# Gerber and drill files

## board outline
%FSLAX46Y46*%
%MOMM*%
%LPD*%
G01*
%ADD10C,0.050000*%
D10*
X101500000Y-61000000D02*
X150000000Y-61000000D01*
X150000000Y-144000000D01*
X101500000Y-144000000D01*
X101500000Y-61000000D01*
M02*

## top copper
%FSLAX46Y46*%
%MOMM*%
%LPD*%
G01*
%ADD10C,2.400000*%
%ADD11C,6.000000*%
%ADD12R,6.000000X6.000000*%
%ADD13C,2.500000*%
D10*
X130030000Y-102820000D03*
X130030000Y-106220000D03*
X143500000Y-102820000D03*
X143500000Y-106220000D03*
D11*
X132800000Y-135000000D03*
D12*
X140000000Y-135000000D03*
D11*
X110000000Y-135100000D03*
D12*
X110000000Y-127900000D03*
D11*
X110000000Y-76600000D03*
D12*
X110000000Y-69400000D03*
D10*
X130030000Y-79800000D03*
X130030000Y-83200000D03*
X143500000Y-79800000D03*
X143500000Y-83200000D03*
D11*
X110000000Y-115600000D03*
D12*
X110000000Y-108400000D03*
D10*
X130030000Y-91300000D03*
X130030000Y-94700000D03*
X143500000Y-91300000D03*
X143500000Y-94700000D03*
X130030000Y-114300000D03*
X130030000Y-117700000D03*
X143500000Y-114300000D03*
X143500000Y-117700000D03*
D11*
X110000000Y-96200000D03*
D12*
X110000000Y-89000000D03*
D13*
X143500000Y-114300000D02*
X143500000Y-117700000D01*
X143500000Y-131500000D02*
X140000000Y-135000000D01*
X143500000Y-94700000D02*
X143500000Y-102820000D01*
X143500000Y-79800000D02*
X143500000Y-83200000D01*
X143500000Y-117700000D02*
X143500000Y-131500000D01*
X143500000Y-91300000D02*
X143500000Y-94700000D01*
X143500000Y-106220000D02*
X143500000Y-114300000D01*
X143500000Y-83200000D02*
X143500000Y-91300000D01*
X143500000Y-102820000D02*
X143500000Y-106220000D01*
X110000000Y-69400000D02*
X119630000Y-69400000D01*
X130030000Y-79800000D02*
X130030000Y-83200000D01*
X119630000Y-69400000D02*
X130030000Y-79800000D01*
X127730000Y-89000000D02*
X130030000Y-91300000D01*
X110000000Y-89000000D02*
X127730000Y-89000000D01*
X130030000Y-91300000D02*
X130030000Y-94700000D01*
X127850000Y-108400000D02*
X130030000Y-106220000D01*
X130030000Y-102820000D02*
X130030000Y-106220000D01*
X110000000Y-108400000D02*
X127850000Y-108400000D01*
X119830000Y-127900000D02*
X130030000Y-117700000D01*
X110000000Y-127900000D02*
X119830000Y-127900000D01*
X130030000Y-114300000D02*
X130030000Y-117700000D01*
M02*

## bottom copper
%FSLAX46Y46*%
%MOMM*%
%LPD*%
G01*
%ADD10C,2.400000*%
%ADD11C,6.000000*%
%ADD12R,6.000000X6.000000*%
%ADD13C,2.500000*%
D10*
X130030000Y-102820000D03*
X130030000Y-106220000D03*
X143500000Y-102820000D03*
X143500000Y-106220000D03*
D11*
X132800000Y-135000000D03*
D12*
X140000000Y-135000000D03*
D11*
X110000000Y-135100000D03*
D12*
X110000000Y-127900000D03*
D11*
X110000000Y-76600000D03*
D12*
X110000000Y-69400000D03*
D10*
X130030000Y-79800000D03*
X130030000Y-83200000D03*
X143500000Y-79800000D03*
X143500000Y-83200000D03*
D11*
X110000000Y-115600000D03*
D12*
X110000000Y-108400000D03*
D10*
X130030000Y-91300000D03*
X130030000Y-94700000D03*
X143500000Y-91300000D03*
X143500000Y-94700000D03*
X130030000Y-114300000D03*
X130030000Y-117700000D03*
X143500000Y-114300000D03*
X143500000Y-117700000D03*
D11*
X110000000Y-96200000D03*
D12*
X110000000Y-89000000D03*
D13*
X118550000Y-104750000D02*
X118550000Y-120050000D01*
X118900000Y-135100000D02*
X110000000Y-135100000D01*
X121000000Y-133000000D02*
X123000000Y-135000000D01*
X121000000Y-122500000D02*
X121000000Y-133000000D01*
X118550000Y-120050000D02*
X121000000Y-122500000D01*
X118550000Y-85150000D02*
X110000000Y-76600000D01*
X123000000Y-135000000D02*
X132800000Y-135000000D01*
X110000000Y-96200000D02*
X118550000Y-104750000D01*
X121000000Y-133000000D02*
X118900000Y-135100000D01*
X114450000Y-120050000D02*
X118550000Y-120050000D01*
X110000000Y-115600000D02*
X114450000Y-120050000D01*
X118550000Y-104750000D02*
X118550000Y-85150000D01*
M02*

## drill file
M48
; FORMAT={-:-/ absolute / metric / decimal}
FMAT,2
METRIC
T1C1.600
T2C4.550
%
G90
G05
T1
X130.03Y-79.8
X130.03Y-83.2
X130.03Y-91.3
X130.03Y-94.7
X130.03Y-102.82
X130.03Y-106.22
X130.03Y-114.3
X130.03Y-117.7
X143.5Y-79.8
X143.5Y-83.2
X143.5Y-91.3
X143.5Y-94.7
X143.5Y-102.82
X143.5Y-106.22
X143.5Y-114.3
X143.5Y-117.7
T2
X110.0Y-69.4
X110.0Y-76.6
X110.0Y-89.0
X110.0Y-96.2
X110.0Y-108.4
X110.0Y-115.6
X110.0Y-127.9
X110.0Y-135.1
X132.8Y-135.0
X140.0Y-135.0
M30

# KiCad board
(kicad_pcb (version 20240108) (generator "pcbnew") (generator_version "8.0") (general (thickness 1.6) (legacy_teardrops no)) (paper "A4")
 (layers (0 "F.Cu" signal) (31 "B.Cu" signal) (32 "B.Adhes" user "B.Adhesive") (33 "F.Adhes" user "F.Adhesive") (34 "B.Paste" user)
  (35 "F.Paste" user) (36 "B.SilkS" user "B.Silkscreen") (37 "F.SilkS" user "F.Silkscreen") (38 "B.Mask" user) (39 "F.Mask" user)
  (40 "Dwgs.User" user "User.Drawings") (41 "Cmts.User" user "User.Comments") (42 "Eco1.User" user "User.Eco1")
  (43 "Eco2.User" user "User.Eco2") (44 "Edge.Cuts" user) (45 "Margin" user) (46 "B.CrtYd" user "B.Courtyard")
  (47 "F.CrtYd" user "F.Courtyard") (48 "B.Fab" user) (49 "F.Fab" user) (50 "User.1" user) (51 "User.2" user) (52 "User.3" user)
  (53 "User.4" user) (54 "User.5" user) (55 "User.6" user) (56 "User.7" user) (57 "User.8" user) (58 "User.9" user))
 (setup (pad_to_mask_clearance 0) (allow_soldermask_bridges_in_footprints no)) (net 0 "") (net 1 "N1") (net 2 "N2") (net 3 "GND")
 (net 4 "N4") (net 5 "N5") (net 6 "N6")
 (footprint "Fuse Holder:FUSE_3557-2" (layer "F.Cu") (at 136.765 104.52)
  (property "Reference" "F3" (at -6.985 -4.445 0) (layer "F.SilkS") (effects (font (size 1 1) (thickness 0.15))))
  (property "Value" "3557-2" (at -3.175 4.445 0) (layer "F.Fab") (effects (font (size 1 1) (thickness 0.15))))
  (pad "1_1" thru_hole circle (at -6.735 -1.7) (size 2.4 2.4) (drill 1.6) (layers "*.Cu" "*.Mask") (remove_unused_layers no) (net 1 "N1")
   (solder_mask_margin 0.102))
  (pad "1_2" thru_hole circle (at -6.735 1.7) (size 2.4 2.4) (drill 1.6) (layers "*.Cu" "*.Mask") (remove_unused_layers no) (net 1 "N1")
   (solder_mask_margin 0.102))
  (pad "2_1" thru_hole circle (at 6.735 -1.7) (size 2.4 2.4) (drill 1.6) (layers "*.Cu" "*.Mask") (remove_unused_layers no) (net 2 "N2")
   (solder_mask_margin 0.102))
  (pad "2_2" thru_hole circle (at 6.735 1.7) (size 2.4 2.4) (drill 1.6) (layers "*.Cu" "*.Mask") (remove_unused_layers no) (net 2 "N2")
   (solder_mask_margin 0.102)))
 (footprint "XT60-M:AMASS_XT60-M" (layer "F.Cu") (at 136.4 135 180)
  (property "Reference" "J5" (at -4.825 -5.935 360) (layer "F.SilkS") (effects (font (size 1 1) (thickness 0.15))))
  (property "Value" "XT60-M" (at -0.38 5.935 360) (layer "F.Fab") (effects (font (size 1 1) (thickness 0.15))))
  (pad "N" thru_hole circle (at 3.6 0 180) (size 6 6) (drill 4.55) (layers "*.Cu" "*.Mask") (remove_unused_layers no) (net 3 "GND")
   (solder_mask_margin 0.102))
  (pad "P" thru_hole rect (at -3.6 0 180) (size 6 6) (drill 4.55) (layers "*.Cu" "*.Mask") (remove_unused_layers no) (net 2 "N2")
   (solder_mask_margin 0.102)))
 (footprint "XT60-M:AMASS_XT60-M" (layer "F.Cu") (at 110 131.5 -90)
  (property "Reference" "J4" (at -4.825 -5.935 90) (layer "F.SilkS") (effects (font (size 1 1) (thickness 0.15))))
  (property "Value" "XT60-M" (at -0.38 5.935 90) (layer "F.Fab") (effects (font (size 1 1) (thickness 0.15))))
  (pad "N" thru_hole circle (at 3.6 0 270) (size 6 6) (drill 4.55) (layers "*.Cu" "*.Mask") (remove_unused_layers no) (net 3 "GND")
   (solder_mask_margin 0.102))
  (pad "P" thru_hole rect (at -3.6 0 270) (size 6 6) (drill 4.55) (layers "*.Cu" "*.Mask") (remove_unused_layers no) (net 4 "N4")
   (solder_mask_margin 0.102)))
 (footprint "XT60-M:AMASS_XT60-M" (layer "F.Cu") (at 110 73 -90)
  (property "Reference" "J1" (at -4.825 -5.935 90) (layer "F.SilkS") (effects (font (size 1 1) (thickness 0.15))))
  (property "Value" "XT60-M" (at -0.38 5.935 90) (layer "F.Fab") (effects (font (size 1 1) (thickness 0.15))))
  (pad "N" thru_hole circle (at 3.6 0 270) (size 6 6) (drill 4.55) (layers "*.Cu" "*.Mask") (remove_unused_layers no) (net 3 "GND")
   (solder_mask_margin 0.102))
  (pad "P" thru_hole rect (at -3.6 0 270) (size 6 6) (drill 4.55) (layers "*.Cu" "*.Mask") (remove_unused_layers no) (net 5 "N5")
   (solder_mask_margin 0.102)))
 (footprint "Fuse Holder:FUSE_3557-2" (layer "F.Cu") (at 136.765 81.5)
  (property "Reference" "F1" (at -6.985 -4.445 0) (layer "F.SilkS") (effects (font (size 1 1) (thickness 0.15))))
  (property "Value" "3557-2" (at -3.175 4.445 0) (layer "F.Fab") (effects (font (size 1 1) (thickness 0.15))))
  (pad "1_1" thru_hole circle (at -6.735 -1.7) (size 2.4 2.4) (drill 1.6) (layers "*.Cu" "*.Mask") (remove_unused_layers no) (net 5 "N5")
   (solder_mask_margin 0.102))
  (pad "1_2" thru_hole circle (at -6.735 1.7) (size 2.4 2.4) (drill 1.6) (layers "*.Cu" "*.Mask") (remove_unused_layers no) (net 5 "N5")
   (solder_mask_margin 0.102))
  (pad "2_1" thru_hole circle (at 6.735 -1.7) (size 2.4 2.4) (drill 1.6) (layers "*.Cu" "*.Mask") (remove_unused_layers no) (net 2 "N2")
   (solder_mask_margin 0.102))
  (pad "2_2" thru_hole circle (at 6.735 1.7) (size 2.4 2.4) (drill 1.6) (layers "*.Cu" "*.Mask") (remove_unused_layers no) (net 2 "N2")
   (solder_mask_margin 0.102)))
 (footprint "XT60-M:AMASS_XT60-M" (layer "F.Cu") (at 110 112 -90)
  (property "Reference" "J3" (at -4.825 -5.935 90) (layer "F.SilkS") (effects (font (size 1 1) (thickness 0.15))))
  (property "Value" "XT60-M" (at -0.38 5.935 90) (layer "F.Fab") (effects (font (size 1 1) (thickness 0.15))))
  (pad "N" thru_hole circle (at 3.6 0 270) (size 6 6) (drill 4.55) (layers "*.Cu" "*.Mask") (remove_unused_layers no) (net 3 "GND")
   (solder_mask_margin 0.102))
  (pad "P" thru_hole rect (at -3.6 0 270) (size 6 6) (drill 4.55) (layers "*.Cu" "*.Mask") (remove_unused_layers no) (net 1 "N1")
   (solder_mask_margin 0.102)))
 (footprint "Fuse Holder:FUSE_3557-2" (layer "F.Cu") (at 136.765 93)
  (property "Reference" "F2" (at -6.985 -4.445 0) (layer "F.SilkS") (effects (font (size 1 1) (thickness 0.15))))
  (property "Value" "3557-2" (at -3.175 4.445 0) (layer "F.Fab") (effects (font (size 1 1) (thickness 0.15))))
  (pad "1_1" thru_hole circle (at -6.735 -1.7) (size 2.4 2.4) (drill 1.6) (layers "*.Cu" "*.Mask") (remove_unused_layers no) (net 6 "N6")
   (solder_mask_margin 0.102))
  (pad "1_2" thru_hole circle (at -6.735 1.7) (size 2.4 2.4) (drill 1.6) (layers "*.Cu" "*.Mask") (remove_unused_layers no) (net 6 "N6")
   (solder_mask_margin 0.102))
  (pad "2_1" thru_hole circle (at 6.735 -1.7) (size 2.4 2.4) (drill 1.6) (layers "*.Cu" "*.Mask") (remove_unused_layers no) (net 2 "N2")
   (solder_mask_margin 0.102))
  (pad "2_2" thru_hole circle (at 6.735 1.7) (size 2.4 2.4) (drill 1.6) (layers "*.Cu" "*.Mask") (remove_unused_layers no) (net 2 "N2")
   (solder_mask_margin 0.102)))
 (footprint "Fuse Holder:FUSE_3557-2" (layer "F.Cu") (at 136.765 116)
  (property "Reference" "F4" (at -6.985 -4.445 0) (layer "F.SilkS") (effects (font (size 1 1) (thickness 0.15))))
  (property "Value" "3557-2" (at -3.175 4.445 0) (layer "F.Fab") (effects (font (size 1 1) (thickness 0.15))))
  (pad "1_1" thru_hole circle (at -6.735 -1.7) (size 2.4 2.4) (drill 1.6) (layers "*.Cu" "*.Mask") (remove_unused_layers no) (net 4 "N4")
   (solder_mask_margin 0.102))
  (pad "1_2" thru_hole circle (at -6.735 1.7) (size 2.4 2.4) (drill 1.6) (layers "*.Cu" "*.Mask") (remove_unused_layers no) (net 4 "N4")
   (solder_mask_margin 0.102))
  (pad "2_1" thru_hole circle (at 6.735 -1.7) (size 2.4 2.4) (drill 1.6) (layers "*.Cu" "*.Mask") (remove_unused_layers no) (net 2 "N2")
   (solder_mask_margin 0.102))
  (pad "2_2" thru_hole circle (at 6.735 1.7) (size 2.4 2.4) (drill 1.6) (layers "*.Cu" "*.Mask") (remove_unused_layers no) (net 2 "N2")
   (solder_mask_margin 0.102)))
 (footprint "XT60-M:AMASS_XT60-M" (layer "F.Cu") (at 110 92.6 -90)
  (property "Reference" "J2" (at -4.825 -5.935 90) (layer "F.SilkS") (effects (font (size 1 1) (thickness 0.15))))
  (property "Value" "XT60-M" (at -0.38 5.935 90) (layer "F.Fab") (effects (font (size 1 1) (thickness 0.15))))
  (pad "N" thru_hole circle (at 3.6 0 270) (size 6 6) (drill 4.55) (layers "*.Cu" "*.Mask") (remove_unused_layers no) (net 3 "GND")
   (solder_mask_margin 0.102))
  (pad "P" thru_hole rect (at -3.6 0 270) (size 6 6) (drill 4.55) (layers "*.Cu" "*.Mask") (remove_unused_layers no) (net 6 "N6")
   (solder_mask_margin 0.102)))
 (gr_poly (pts (xy 101.5 61) (xy 150 61) (xy 150 144) (xy 101.5 144)) (stroke (width 0.05) (type solid)) (fill none) (layer "Edge.Cuts"))
 (segment (start 143.5 114.3) (end 143.5 117.7) (width 2.5) (layer "F.Cu") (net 2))
 (segment (start 143.5 131.5) (end 140 135) (width 2.5) (layer "F.Cu") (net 2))
 (segment (start 143.5 94.7) (end 143.5 102.82) (width 2.5) (layer "F.Cu") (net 2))
 (segment (start 143.5 79.8) (end 143.5 83.2) (width 2.5) (layer "F.Cu") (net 2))
 (segment (start 143.5 117.7) (end 143.5 131.5) (width 2.5) (layer "F.Cu") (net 2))
 (segment (start 143.5 91.3) (end 143.5 94.7) (width 2.5) (layer "F.Cu") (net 2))
 (segment (start 143.5 106.22) (end 143.5 114.3) (width 2.5) (layer "F.Cu") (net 2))
 (segment (start 143.5 83.2) (end 143.5 91.3) (width 2.5) (layer "F.Cu") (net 2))
 (segment (start 143.5 102.82) (end 143.5 106.22) (width 2.5) (layer "F.Cu") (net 2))
 (segment (start 110 69.4) (end 119.63 69.4) (width 2.5) (layer "F.Cu") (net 5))
 (segment (start 130.03 79.8) (end 130.03 83.2) (width 2.5) (layer "F.Cu") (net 5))
 (segment (start 119.63 69.4) (end 130.03 79.8) (width 2.5) (layer "F.Cu") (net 5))
 (segment (start 127.73 89) (end 130.03 91.3) (width 2.5) (layer "F.Cu") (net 6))
 (segment (start 110 89) (end 127.73 89) (width 2.5) (layer "F.Cu") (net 6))
 (segment (start 130.03 91.3) (end 130.03 94.7) (width 2.5) (layer "F.Cu") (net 6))
 (segment (start 127.85 108.4) (end 130.03 106.22) (width 2.5) (layer "F.Cu") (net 1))
 (segment (start 130.03 102.82) (end 130.03 106.22) (width 2.5) (layer "F.Cu") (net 1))
 (segment (start 110 108.4) (end 127.85 108.4) (width 2.5) (layer "F.Cu") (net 1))
 (segment (start 119.83 127.9) (end 130.03 117.7) (width 2.5) (layer "F.Cu") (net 4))
 (segment (start 110 127.9) (end 119.83 127.9) (width 2.5) (layer "F.Cu") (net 4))
 (segment (start 130.03 114.3) (end 130.03 117.7) (width 2.5) (layer "F.Cu") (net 4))
 (segment (start 118.55 104.75) (end 118.55 120.05) (width 2.5) (layer "B.Cu") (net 3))
 (segment (start 118.9 135.1) (end 110 135.1) (width 2.5) (layer "B.Cu") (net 3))
 (segment (start 121 133) (end 123 135) (width 2.5) (layer "B.Cu") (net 3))
 (segment (start 121 122.5) (end 121 133) (width 2.5) (layer "B.Cu") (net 3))
 (segment (start 118.55 120.05) (end 121 122.5) (width 2.5) (layer "B.Cu") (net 3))
 (segment (start 118.55 85.15) (end 110 76.6) (width 2.5) (layer "B.Cu") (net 3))
 (segment (start 123 135) (end 132.8 135) (width 2.5) (layer "B.Cu") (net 3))
 (segment (start 110 96.2) (end 118.55 104.75) (width 2.5) (layer "B.Cu") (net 3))
 (segment (start 121 133) (end 118.9 135.1) (width 2.5) (layer "B.Cu") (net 3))
 (segment (start 114.45 120.05) (end 118.55 120.05) (width 2.5) (layer "B.Cu") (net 3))
 (segment (start 110 115.6) (end 114.45 120.05) (width 2.5) (layer "B.Cu") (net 3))
 (segment (start 118.55 104.75) (end 118.55 85.15) (width 2.5) (layer "B.Cu") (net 3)))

